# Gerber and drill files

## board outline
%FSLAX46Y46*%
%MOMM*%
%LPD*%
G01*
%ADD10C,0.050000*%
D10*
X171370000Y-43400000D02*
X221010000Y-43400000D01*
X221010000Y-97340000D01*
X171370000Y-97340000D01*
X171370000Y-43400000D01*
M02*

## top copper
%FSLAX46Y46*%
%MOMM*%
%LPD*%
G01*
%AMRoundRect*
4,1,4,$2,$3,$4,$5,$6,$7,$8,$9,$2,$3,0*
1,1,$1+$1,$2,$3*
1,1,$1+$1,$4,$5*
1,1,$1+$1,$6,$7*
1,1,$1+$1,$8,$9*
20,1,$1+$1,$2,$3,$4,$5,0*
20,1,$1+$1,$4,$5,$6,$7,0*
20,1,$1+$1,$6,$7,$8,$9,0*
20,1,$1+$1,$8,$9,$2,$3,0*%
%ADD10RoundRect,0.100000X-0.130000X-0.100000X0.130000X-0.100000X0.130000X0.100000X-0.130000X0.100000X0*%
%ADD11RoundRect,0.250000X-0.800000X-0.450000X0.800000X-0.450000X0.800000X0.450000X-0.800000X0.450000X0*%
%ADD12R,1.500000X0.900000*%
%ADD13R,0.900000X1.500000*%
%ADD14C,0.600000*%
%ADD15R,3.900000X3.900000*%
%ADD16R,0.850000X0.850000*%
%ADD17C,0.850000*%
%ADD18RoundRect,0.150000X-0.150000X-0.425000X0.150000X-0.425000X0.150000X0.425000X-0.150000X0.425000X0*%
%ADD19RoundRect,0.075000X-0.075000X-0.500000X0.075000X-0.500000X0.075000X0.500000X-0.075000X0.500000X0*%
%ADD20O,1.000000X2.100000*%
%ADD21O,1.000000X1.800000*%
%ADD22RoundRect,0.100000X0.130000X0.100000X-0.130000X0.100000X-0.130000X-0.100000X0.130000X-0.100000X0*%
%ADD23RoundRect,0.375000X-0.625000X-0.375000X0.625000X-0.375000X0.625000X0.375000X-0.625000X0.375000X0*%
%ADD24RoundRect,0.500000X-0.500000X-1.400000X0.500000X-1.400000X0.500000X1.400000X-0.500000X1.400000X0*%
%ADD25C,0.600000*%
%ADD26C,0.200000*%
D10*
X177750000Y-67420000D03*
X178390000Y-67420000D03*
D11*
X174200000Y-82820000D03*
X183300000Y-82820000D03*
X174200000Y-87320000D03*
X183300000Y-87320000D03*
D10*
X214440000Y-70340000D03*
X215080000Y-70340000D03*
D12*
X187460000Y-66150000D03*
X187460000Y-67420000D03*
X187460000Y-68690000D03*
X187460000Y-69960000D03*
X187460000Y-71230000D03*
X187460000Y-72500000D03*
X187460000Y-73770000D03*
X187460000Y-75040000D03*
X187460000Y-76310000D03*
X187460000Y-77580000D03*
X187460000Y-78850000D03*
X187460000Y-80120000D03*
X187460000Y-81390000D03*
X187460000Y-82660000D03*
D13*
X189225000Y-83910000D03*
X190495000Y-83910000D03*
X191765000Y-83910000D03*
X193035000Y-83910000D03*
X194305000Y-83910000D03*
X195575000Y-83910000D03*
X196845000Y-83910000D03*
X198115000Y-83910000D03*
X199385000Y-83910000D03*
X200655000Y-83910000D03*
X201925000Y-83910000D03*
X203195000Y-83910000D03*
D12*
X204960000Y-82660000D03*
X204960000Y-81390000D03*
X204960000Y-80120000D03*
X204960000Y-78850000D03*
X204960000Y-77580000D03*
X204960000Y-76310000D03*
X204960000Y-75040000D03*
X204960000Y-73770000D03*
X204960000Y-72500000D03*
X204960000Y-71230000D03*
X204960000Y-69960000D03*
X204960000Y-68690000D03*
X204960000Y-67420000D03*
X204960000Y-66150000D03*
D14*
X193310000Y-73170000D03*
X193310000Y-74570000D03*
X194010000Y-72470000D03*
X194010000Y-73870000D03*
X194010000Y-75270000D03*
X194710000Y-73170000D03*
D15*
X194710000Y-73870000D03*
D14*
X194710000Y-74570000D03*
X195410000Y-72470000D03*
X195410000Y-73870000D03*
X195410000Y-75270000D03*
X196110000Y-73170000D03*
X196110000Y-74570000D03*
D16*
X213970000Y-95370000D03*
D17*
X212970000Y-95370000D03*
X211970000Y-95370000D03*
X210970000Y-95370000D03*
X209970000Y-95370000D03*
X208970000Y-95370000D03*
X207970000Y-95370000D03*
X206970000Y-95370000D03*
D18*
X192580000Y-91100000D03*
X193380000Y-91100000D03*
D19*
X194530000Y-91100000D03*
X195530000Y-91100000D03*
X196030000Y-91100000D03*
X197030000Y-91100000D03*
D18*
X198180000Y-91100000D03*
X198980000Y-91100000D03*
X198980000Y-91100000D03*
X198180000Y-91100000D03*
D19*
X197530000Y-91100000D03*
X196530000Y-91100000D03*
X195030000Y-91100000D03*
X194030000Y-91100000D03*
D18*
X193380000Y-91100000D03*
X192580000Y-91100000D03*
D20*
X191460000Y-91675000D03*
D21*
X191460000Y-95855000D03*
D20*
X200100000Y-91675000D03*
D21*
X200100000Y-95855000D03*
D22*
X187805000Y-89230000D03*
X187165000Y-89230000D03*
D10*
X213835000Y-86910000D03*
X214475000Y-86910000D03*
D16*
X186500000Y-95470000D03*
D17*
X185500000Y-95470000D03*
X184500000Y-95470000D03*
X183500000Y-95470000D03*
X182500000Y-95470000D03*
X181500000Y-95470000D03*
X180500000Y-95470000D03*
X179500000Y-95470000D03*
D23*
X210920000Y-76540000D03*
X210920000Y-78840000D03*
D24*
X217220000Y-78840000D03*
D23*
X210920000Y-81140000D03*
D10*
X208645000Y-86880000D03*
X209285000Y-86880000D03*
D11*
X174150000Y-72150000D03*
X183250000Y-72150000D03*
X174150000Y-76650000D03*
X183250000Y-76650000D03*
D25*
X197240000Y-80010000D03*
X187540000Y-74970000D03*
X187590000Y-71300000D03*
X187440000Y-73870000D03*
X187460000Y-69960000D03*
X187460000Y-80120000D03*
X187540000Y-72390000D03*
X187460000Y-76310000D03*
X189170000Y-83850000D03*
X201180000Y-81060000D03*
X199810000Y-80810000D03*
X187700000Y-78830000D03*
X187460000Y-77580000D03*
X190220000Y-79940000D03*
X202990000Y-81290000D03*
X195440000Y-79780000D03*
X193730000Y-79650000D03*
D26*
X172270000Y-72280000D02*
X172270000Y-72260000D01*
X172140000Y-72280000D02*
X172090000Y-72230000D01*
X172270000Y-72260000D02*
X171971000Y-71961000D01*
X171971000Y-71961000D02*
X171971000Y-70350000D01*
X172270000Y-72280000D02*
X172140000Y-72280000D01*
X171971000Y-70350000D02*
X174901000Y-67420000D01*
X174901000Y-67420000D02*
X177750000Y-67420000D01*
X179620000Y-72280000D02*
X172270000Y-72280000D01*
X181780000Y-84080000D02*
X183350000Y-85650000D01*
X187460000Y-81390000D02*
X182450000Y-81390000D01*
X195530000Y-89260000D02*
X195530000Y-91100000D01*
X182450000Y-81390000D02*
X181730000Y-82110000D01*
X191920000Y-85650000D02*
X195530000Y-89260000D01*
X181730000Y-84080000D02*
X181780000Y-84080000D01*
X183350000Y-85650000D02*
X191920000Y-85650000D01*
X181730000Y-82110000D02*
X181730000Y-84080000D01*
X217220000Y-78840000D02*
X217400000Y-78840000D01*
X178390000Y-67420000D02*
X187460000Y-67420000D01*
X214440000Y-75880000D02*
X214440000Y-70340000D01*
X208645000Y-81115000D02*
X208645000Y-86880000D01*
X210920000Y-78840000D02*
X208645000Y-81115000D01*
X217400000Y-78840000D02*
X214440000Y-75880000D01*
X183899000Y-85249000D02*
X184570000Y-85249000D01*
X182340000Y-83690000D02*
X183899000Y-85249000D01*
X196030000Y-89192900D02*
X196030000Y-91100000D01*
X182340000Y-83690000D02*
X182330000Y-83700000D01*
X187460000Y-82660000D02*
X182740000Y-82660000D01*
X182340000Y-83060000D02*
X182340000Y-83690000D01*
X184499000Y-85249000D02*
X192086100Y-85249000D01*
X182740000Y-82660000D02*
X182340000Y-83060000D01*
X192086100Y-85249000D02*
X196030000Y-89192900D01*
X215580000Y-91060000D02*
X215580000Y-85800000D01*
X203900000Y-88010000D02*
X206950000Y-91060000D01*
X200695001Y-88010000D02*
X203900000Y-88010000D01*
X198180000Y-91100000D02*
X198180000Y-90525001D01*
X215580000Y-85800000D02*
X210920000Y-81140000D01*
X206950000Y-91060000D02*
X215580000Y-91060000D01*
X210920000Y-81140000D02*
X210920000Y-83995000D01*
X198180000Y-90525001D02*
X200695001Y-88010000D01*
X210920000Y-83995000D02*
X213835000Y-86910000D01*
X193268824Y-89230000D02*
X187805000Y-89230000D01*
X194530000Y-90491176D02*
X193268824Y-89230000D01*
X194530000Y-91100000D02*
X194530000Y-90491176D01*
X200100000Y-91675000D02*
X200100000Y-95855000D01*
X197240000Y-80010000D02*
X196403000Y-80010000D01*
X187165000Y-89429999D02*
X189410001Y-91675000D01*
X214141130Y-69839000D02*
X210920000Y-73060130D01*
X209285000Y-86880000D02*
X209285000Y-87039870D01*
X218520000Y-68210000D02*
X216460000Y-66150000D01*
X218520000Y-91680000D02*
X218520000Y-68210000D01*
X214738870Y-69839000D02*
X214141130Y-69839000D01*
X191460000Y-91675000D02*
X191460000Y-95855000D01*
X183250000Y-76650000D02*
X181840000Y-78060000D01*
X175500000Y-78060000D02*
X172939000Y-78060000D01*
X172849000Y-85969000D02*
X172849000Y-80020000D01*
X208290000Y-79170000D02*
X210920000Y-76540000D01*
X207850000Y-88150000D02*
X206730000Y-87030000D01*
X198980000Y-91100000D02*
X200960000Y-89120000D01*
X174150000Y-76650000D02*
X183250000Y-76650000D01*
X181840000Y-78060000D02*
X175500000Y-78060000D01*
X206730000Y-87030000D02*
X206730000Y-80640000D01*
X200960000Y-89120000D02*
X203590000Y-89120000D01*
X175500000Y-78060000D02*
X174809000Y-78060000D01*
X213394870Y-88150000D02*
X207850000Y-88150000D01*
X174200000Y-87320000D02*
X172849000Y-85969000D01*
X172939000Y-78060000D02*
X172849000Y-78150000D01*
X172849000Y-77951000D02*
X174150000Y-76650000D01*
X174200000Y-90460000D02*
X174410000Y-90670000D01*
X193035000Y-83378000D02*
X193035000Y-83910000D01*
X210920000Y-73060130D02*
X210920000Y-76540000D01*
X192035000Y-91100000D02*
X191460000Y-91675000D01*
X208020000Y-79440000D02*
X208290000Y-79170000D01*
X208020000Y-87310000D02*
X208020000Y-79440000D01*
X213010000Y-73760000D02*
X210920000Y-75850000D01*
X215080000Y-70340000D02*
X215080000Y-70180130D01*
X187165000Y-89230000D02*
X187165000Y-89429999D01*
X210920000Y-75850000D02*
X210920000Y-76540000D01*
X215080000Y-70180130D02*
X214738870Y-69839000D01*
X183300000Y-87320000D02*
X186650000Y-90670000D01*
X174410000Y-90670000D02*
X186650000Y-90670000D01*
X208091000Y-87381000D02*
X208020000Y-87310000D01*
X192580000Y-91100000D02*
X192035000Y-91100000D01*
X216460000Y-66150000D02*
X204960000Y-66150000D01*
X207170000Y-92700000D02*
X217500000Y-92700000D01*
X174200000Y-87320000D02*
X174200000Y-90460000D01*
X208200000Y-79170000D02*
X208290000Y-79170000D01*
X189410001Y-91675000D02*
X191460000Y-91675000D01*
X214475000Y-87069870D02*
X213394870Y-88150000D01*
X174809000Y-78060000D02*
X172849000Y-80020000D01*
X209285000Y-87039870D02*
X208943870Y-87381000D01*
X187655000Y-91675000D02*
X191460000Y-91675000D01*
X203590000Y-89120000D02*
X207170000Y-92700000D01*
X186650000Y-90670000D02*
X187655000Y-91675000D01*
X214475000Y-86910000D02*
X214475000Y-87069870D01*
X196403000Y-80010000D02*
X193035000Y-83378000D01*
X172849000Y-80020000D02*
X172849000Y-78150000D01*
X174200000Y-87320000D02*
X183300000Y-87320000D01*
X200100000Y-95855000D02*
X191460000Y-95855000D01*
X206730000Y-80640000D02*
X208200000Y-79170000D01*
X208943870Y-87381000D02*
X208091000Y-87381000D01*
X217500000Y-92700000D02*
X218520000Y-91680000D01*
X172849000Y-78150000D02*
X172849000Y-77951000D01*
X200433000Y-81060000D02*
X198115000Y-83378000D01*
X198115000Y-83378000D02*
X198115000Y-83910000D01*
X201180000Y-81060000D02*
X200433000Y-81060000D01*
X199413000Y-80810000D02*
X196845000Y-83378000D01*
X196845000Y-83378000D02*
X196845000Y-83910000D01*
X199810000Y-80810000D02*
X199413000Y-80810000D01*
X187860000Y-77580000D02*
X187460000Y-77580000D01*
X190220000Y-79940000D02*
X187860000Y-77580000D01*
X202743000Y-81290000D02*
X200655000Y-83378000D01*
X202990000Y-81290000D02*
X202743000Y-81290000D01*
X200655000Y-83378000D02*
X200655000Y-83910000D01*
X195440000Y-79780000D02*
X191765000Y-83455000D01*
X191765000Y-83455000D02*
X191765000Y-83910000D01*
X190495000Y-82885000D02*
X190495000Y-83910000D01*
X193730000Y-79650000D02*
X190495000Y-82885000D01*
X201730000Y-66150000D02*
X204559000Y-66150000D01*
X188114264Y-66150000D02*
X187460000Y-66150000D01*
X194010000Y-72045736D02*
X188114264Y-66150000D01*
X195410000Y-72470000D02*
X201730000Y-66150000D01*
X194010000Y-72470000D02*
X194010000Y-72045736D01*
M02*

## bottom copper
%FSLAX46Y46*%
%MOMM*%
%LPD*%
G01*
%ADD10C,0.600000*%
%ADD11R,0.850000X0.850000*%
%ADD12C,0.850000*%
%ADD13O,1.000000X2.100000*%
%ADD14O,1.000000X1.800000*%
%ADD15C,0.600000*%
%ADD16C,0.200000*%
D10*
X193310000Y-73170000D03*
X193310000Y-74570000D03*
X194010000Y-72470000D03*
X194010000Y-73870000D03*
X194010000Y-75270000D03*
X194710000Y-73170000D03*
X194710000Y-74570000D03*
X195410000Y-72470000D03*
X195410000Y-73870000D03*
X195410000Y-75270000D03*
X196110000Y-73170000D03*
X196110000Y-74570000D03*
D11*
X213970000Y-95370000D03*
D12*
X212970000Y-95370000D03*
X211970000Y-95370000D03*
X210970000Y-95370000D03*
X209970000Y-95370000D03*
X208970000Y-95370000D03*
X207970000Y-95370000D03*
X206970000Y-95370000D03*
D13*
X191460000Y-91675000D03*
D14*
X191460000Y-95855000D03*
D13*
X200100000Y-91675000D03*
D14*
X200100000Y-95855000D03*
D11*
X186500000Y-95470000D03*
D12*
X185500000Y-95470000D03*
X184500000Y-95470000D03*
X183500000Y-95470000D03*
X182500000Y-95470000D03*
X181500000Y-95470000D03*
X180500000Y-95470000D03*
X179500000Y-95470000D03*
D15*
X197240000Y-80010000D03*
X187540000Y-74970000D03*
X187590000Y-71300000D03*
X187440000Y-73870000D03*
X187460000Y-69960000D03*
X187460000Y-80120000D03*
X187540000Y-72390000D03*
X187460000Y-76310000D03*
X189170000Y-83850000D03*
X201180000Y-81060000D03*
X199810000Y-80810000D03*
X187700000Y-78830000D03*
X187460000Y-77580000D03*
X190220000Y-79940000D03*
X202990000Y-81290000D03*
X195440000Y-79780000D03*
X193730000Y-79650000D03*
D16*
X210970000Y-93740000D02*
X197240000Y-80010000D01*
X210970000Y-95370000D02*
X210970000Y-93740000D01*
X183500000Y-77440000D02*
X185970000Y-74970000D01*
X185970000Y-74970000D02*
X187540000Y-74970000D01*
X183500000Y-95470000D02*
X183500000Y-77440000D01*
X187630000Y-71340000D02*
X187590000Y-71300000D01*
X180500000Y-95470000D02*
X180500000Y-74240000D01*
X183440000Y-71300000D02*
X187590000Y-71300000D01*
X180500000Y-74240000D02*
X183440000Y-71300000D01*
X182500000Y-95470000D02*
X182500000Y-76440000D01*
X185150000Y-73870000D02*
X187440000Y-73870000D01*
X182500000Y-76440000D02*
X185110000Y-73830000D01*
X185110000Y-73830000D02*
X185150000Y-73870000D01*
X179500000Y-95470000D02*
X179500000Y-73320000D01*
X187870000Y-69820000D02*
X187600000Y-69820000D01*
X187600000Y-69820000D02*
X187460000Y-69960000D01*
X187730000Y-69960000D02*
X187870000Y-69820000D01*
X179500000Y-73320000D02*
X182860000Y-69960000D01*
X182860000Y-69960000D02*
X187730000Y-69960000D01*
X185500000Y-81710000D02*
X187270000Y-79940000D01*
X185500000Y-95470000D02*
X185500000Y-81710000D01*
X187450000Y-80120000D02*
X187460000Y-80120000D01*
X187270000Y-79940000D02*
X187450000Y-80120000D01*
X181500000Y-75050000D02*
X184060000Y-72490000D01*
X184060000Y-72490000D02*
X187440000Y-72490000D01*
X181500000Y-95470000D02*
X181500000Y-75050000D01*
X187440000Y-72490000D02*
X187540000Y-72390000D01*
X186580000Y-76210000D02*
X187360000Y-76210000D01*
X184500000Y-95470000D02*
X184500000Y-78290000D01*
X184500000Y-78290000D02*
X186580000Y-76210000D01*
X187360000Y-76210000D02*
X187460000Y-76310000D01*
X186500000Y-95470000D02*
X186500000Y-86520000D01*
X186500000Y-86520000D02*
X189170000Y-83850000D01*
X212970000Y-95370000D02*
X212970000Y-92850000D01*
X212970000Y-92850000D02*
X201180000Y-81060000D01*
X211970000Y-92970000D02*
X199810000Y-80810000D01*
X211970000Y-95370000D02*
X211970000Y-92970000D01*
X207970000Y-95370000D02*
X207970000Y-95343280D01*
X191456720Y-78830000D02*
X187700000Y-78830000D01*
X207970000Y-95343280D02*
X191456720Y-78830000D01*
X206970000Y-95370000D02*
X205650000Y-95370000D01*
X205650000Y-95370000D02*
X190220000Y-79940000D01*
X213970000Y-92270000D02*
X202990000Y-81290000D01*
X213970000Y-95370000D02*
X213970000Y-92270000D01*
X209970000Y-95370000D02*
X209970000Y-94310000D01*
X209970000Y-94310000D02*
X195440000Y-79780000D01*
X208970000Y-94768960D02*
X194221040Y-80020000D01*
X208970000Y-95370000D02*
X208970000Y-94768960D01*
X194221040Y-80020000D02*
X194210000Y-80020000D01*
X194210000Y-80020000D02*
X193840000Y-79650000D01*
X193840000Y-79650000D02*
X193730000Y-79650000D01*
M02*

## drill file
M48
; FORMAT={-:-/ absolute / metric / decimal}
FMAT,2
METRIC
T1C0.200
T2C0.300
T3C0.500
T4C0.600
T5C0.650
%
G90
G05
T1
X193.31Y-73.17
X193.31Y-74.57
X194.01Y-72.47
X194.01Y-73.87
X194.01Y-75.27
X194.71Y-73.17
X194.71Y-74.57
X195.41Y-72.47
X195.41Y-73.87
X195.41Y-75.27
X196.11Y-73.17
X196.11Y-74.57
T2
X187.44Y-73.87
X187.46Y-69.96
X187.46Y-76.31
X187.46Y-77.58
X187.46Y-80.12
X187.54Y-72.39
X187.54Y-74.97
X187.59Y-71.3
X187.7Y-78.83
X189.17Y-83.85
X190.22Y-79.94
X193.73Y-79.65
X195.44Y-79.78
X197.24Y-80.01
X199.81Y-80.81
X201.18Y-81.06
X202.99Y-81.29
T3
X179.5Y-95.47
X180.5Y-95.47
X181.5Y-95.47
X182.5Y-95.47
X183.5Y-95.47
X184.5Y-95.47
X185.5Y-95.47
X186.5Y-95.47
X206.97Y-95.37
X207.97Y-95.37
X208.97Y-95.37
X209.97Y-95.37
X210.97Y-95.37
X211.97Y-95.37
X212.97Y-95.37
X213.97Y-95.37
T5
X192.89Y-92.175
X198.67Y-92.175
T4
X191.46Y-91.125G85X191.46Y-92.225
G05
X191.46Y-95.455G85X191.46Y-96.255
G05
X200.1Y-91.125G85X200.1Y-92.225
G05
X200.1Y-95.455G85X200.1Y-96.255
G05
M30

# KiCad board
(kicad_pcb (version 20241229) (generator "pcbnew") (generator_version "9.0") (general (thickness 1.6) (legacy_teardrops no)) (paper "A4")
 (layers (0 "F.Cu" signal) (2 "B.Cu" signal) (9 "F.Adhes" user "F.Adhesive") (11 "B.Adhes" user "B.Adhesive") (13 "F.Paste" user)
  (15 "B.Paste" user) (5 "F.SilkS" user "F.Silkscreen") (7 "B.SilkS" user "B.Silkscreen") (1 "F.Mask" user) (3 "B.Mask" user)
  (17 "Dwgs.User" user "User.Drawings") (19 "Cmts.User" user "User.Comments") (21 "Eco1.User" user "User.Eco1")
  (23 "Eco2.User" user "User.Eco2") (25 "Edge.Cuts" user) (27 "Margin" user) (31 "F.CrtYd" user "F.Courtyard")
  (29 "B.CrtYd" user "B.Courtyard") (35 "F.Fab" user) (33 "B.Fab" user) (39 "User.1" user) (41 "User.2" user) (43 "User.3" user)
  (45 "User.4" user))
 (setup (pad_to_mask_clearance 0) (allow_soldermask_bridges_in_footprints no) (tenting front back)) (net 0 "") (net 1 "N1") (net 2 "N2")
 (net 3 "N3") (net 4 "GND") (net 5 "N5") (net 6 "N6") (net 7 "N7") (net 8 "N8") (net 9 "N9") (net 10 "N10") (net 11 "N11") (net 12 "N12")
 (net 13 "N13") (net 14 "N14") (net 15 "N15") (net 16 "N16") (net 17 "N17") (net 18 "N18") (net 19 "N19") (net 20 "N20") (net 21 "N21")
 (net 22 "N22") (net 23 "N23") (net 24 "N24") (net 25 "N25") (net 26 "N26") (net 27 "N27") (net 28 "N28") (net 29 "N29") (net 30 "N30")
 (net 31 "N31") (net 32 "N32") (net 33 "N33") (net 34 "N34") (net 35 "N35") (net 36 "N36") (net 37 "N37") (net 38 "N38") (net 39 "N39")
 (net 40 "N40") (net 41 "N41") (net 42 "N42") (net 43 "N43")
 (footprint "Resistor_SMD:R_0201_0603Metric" (layer "F.Cu") (at 178.07 67.42)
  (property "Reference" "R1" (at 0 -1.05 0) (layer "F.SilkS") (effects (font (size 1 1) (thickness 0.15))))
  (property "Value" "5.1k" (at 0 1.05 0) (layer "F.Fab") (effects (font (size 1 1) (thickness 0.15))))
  (pad "" smd roundrect (at -0.345 0) (size 0.318 0.36) (layers "F.Paste") (roundrect_rratio 0.25))
  (pad "" smd roundrect (at 0.345 0) (size 0.318 0.36) (layers "F.Paste") (roundrect_rratio 0.25))
  (pad "1" smd roundrect (at -0.32 0) (size 0.46 0.4) (layers "F.Cu" "F.Mask") (roundrect_rratio 0.25) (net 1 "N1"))
  (pad "2" smd roundrect (at 0.32 0) (size 0.46 0.4) (layers "F.Cu" "F.Mask") (roundrect_rratio 0.25) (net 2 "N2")))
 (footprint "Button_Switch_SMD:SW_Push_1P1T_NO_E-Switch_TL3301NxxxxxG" (layer "F.Cu") (at 178.75 85.07)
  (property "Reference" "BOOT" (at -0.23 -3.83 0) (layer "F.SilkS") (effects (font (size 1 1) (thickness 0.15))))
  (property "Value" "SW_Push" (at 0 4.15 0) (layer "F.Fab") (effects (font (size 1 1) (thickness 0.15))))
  (pad "1" smd roundrect (at -4.55 -2.25) (size 2.1 1.4) (layers "F.Cu" "F.Mask" "F.Paste") (roundrect_rratio 0.1785714286) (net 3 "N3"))
  (pad "1" smd roundrect (at 4.55 -2.25) (size 2.1 1.4) (layers "F.Cu" "F.Mask" "F.Paste") (roundrect_rratio 0.1785714286) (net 3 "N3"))
  (pad "2" smd roundrect (at -4.55 2.25) (size 2.1 1.4) (layers "F.Cu" "F.Mask" "F.Paste") (roundrect_rratio 0.1785714286) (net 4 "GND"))
  (pad "2" smd roundrect (at 4.55 2.25) (size 2.1 1.4) (layers "F.Cu" "F.Mask" "F.Paste") (roundrect_rratio 0.1785714286) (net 4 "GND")))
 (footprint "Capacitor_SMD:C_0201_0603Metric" (layer "F.Cu") (at 214.76 70.34)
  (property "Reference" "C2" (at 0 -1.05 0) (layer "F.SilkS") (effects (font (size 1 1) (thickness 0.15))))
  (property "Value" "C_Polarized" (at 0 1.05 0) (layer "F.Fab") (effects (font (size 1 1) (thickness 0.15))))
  (pad "" smd roundrect (at -0.345 0) (size 0.318 0.36) (layers "F.Paste") (roundrect_rratio 0.25))
  (pad "" smd roundrect (at 0.345 0) (size 0.318 0.36) (layers "F.Paste") (roundrect_rratio 0.25))
  (pad "1" smd roundrect (at -0.32 0) (size 0.46 0.4) (layers "F.Cu" "F.Mask") (roundrect_rratio 0.25) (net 2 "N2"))
  (pad "2" smd roundrect (at 0.32 0) (size 0.46 0.4) (layers "F.Cu" "F.Mask") (roundrect_rratio 0.25) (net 4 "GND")))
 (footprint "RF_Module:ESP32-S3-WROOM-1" (layer "F.Cu") (at 196.21 71.41)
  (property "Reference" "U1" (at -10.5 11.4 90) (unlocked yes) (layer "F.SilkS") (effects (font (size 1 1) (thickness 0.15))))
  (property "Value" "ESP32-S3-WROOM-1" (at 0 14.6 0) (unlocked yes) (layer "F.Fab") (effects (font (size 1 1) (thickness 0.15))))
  (pad "" smd rect (at -2.9 1.06) (size 0.9 0.9) (layers "F.Paste"))
  (pad "" smd rect (at -2.9 2.46 270) (size 0.9 0.9) (layers "F.Paste"))
  (pad "" smd rect (at -2.9 3.86) (size 0.9 0.9) (layers "F.Paste"))
  (pad "" smd rect (at -1.5 1.06 270) (size 0.9 0.9) (layers "F.Paste"))
  (pad "" smd rect (at -1.5 2.46 270) (size 0.9 0.9) (layers "F.Paste"))
  (pad "" smd rect (at -1.5 3.86 270) (size 0.9 0.9) (layers "F.Paste"))
  (pad "" smd rect (at -0.1 1.06 270) (size 0.9 0.9) (layers "F.Paste"))
  (pad "" smd rect (at -0.1 2.46 270) (size 0.9 0.9) (layers "F.Paste"))
  (pad "" smd rect (at -0.1 3.86 270) (size 0.9 0.9) (layers "F.Paste"))
  (pad "1" smd rect (at -8.75 -5.26) (size 1.5 0.9) (layers "F.Cu" "F.Mask" "F.Paste") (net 4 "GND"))
  (pad "2" smd rect (at -8.75 -3.99) (size 1.5 0.9) (layers "F.Cu" "F.Mask" "F.Paste") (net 2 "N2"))
  (pad "3" smd rect (at -8.75 -2.72) (size 1.5 0.9) (layers "F.Cu" "F.Mask" "F.Paste") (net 1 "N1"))
  (pad "4" smd rect (at -8.75 -1.45) (size 1.5 0.9) (layers "F.Cu" "F.Mask" "F.Paste") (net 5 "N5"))
  (pad "5" smd rect (at -8.75 -0.18) (size 1.5 0.9) (layers "F.Cu" "F.Mask" "F.Paste") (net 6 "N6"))
  (pad "6" smd rect (at -8.75 1.09) (size 1.5 0.9) (layers "F.Cu" "F.Mask" "F.Paste") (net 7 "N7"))
  (pad "7" smd rect (at -8.75 2.36) (size 1.5 0.9) (layers "F.Cu" "F.Mask" "F.Paste") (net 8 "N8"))
  (pad "8" smd rect (at -8.75 3.63) (size 1.5 0.9) (layers "F.Cu" "F.Mask" "F.Paste") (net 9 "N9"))
  (pad "9" smd rect (at -8.75 4.9) (size 1.5 0.9) (layers "F.Cu" "F.Mask" "F.Paste") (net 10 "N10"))
  (pad "10" smd rect (at -8.75 6.17) (size 1.5 0.9) (layers "F.Cu" "F.Mask" "F.Paste") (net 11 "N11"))
  (pad "11" smd rect (at -8.75 7.44) (size 1.5 0.9) (layers "F.Cu" "F.Mask" "F.Paste") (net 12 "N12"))
  (pad "12" smd rect (at -8.75 8.71) (size 1.5 0.9) (layers "F.Cu" "F.Mask" "F.Paste") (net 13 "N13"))
  (pad "13" smd rect (at -8.75 9.98) (size 1.5 0.9) (layers "F.Cu" "F.Mask" "F.Paste") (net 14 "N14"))
  (pad "14" smd rect (at -8.75 11.25 180) (size 1.5 0.9) (layers "F.Cu" "F.Mask" "F.Paste") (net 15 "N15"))
  (pad "15" smd rect (at -6.985 12.5 270) (size 1.5 0.9) (layers "F.Cu" "F.Mask" "F.Paste") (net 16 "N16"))
  (pad "16" smd rect (at -5.715 12.5 270) (size 1.5 0.9) (layers "F.Cu" "F.Mask" "F.Paste") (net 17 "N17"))
  (pad "17" smd rect (at -4.445 12.5 270) (size 1.5 0.9) (layers "F.Cu" "F.Mask" "F.Paste") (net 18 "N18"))
  (pad "18" smd rect (at -3.175 12.5 270) (size 1.5 0.9) (layers "F.Cu" "F.Mask" "F.Paste") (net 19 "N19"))
  (pad "19" smd rect (at -1.905 12.5 270) (size 1.5 0.9) (layers "F.Cu" "F.Mask" "F.Paste") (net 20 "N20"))
  (pad "20" smd rect (at -0.635 12.5 270) (size 1.5 0.9) (layers "F.Cu" "F.Mask" "F.Paste") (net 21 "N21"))
  (pad "21" smd rect (at 0.635 12.5 270) (size 1.5 0.9) (layers "F.Cu" "F.Mask" "F.Paste") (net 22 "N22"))
  (pad "22" smd rect (at 1.905 12.5 270) (size 1.5 0.9) (layers "F.Cu" "F.Mask" "F.Paste") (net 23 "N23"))
  (pad "23" smd rect (at 3.175 12.5 270) (size 1.5 0.9) (layers "F.Cu" "F.Mask" "F.Paste") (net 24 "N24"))
  (pad "24" smd rect (at 4.445 12.5 270) (size 1.5 0.9) (layers "F.Cu" "F.Mask" "F.Paste") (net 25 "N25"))
  (pad "25" smd rect (at 5.715 12.5 270) (size 1.5 0.9) (layers "F.Cu" "F.Mask" "F.Paste") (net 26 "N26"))
  (pad "26" smd rect (at 6.985 12.5 270) (size 1.5 0.9) (layers "F.Cu" "F.Mask" "F.Paste") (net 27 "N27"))
  (pad "27" smd rect (at 8.75 11.25) (size 1.5 0.9) (layers "F.Cu" "F.Mask" "F.Paste") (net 3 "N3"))
  (pad "28" smd rect (at 8.75 9.98) (size 1.5 0.9) (layers "F.Cu" "F.Mask" "F.Paste") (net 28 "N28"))
  (pad "29" smd rect (at 8.75 8.71) (size 1.5 0.9) (layers "F.Cu" "F.Mask" "F.Paste") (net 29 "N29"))
  (pad "30" smd rect (at 8.75 7.44) (size 1.5 0.9) (layers "F.Cu" "F.Mask" "F.Paste") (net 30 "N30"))
  (pad "31" smd rect (at 8.75 6.17) (size 1.5 0.9) (layers "F.Cu" "F.Mask" "F.Paste") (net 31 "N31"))
  (pad "32" smd rect (at 8.75 4.9) (size 1.5 0.9) (layers "F.Cu" "F.Mask" "F.Paste") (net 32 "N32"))
  (pad "33" smd rect (at 8.75 3.63) (size 1.5 0.9) (layers "F.Cu" "F.Mask" "F.Paste") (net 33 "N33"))
  (pad "34" smd rect (at 8.75 2.36) (size 1.5 0.9) (layers "F.Cu" "F.Mask" "F.Paste") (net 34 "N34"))
  (pad "35" smd rect (at 8.75 1.09) (size 1.5 0.9) (layers "F.Cu" "F.Mask" "F.Paste") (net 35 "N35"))
  (pad "36" smd rect (at 8.75 -0.18) (size 1.5 0.9) (layers "F.Cu" "F.Mask" "F.Paste") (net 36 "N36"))
  (pad "37" smd rect (at 8.75 -1.45) (size 1.5 0.9) (layers "F.Cu" "F.Mask" "F.Paste") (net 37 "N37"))
  (pad "38" smd rect (at 8.75 -2.72) (size 1.5 0.9) (layers "F.Cu" "F.Mask" "F.Paste") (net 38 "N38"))
  (pad "39" smd rect (at 8.75 -3.99) (size 1.5 0.9) (layers "F.Cu" "F.Mask" "F.Paste") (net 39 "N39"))
  (pad "40" smd rect (at 8.75 -5.26) (size 1.5 0.9) (layers "F.Cu" "F.Mask" "F.Paste") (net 4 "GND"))
  (pad "41" thru_hole circle (at -2.9 1.76 90) (size 0.6 0.6) (drill 0.2) (layers "*.Cu" "F.Mask") (remove_unused_layers no) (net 4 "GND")
   (zone_connect 2))
  (pad "41" thru_hole circle (at -2.9 3.16) (size 0.6 0.6) (drill 0.2) (layers "*.Cu" "F.Mask") (remove_unused_layers no) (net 4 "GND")
   (zone_connect 2))
  (pad "41" thru_hole circle (at -2.2 1.06) (size 0.6 0.6) (drill 0.2) (layers "*.Cu" "F.Mask") (remove_unused_layers no) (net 4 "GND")
   (zone_connect 2))
  (pad "41" thru_hole circle (at -2.2 2.46) (size 0.6 0.6) (drill 0.2) (layers "*.Cu" "F.Mask") (remove_unused_layers no) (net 4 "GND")
   (zone_connect 2))
  (pad "41" thru_hole circle (at -2.2 3.86) (size 0.6 0.6) (drill 0.2) (layers "*.Cu" "F.Mask") (remove_unused_layers no) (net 4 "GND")
   (zone_connect 2))
  (pad "41" thru_hole circle (at -1.5 1.76) (size 0.6 0.6) (drill 0.2) (layers "*.Cu" "F.Mask") (remove_unused_layers no) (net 4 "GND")
   (zone_connect 2))
  (pad "41" smd rect (at -1.5 2.46 270) (size 3.9 3.9) (layers "F.Cu" "F.Mask") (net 4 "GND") (zone_connect 2))
  (pad "41" thru_hole circle (at -1.5 3.16) (size 0.6 0.6) (drill 0.2) (layers "*.Cu" "F.Mask") (remove_unused_layers no) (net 4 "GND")
   (zone_connect 2))
  (pad "41" thru_hole circle (at -0.8 1.06) (size 0.6 0.6) (drill 0.2) (layers "*.Cu" "F.Mask") (remove_unused_layers no) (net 4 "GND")
   (zone_connect 2))
  (pad "41" thru_hole circle (at -0.8 2.46) (size 0.6 0.6) (drill 0.2) (layers "*.Cu" "F.Mask") (remove_unused_layers no) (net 4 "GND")
   (zone_connect 2))
  (pad "41" thru_hole circle (at -0.8 3.86) (size 0.6 0.6) (drill 0.2) (layers "*.Cu" "F.Mask") (remove_unused_layers no) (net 4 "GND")
   (zone_connect 2))
  (pad "41" thru_hole circle (at -0.1 1.76) (size 0.6 0.6) (drill 0.2) (layers "*.Cu" "F.Mask") (remove_unused_layers no) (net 4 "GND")
   (zone_connect 2))
  (pad "41" thru_hole circle (at -0.1 3.16) (size 0.6 0.6) (drill 0.2) (layers "*.Cu" "F.Mask") (remove_unused_layers no) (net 4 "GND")
   (zone_connect 2))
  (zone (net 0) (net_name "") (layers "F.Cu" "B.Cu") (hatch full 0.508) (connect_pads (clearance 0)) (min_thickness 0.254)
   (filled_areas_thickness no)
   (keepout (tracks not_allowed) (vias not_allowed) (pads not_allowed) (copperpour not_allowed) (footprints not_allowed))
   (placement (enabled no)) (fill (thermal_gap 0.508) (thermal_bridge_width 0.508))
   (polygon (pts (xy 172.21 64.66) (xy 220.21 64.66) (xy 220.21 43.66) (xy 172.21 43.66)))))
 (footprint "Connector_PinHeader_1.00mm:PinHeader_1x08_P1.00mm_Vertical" (layer "F.Cu") (at 213.97 95.37 -90)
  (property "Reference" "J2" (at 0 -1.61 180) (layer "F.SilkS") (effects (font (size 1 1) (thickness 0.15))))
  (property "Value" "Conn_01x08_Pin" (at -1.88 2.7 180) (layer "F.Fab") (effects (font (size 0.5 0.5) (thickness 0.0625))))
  (pad "1" thru_hole rect (at 0 0 270) (size 0.85 0.85) (drill 0.5) (layers "*.Cu" "*.Mask") (remove_unused_layers no) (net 25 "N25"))
  (pad "2" thru_hole circle (at 0 1 270) (size 0.85 0.85) (drill 0.5) (layers "*.Cu" "*.Mask") (remove_unused_layers no) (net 23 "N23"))
  (pad "3" thru_hole circle (at 0 2 270) (size 0.85 0.85) (drill 0.5) (layers "*.Cu" "*.Mask") (remove_unused_layers no) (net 22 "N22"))
  (pad "4" thru_hole circle (at 0 3 270) (size 0.85 0.85) (drill 0.5) (layers "*.Cu" "*.Mask") (remove_unused_layers no) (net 19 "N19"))
  (pad "5" thru_hole circle (at 0 4 270) (size 0.85 0.85) (drill 0.5) (layers "*.Cu" "*.Mask") (remove_unused_layers no) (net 18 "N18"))
  (pad "6" thru_hole circle (at 0 5 270) (size 0.85 0.85) (drill 0.5) (layers "*.Cu" "*.Mask") (remove_unused_layers no) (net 17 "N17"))
  (pad "7" thru_hole circle (at 0 6 270) (size 0.85 0.85) (drill 0.5) (layers "*.Cu" "*.Mask") (remove_unused_layers no) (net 12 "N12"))
  (pad "8" thru_hole circle (at 0 7 270) (size 0.85 0.85) (drill 0.5) (layers "*.Cu" "*.Mask") (remove_unused_layers no) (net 11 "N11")))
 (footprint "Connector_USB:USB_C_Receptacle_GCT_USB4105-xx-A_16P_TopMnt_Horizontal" (layer "F.Cu") (at 195.78 94.78)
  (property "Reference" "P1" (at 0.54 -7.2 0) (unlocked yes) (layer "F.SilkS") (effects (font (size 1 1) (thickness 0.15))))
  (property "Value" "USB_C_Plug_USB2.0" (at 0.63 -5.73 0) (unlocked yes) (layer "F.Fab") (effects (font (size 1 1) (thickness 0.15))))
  (pad "" np_thru_hole circle (at -2.89 -2.605) (size 0.65 0.65) (drill 0.65) (layers "*.Cu" "*.Mask"))
  (pad "" np_thru_hole circle (at 2.89 -2.605) (size 0.65 0.65) (drill 0.65) (layers "*.Cu" "*.Mask"))
  (pad "A1" smd roundrect (at -3.2 -3.68) (size 0.6 1.15) (layers "F.Cu" "F.Mask" "F.Paste") (roundrect_rratio 0.25) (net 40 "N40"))
  (pad "A4" smd roundrect (at -2.4 -3.68) (size 0.6 1.15) (layers "F.Cu" "F.Mask" "F.Paste") (roundrect_rratio 0.25) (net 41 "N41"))
  (pad "A5" smd roundrect (at -1.25 -3.68) (size 0.3 1.15) (layers "F.Cu" "F.Mask" "F.Paste") (roundrect_rratio 0.25) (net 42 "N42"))
  (pad "A6" smd roundrect (at -0.25 -3.68) (size 0.3 1.15) (layers "F.Cu" "F.Mask" "F.Paste") (roundrect_rratio 0.25) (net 14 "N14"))
  (pad "A7" smd roundrect (at 0.25 -3.68) (size 0.3 1.15) (layers "F.Cu" "F.Mask" "F.Paste") (roundrect_rratio 0.25) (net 15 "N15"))
  (pad "A8" smd roundrect (at 1.25 -3.68) (size 0.3 1.15) (layers "F.Cu" "F.Mask" "F.Paste") (roundrect_rratio 0.25))
  (pad "A9" smd roundrect (at 2.4 -3.68) (size 0.6 1.15) (layers "F.Cu" "F.Mask" "F.Paste") (roundrect_rratio 0.25) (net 41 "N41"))
  (pad "A12" smd roundrect (at 3.2 -3.68) (size 0.6 1.15) (layers "F.Cu" "F.Mask" "F.Paste") (roundrect_rratio 0.25) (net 40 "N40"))
  (pad "B1" smd roundrect (at 3.2 -3.68) (size 0.6 1.15) (layers "F.Cu" "F.Mask" "F.Paste") (roundrect_rratio 0.25) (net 40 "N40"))
  (pad "B4" smd roundrect (at 2.4 -3.68) (size 0.6 1.15) (layers "F.Cu" "F.Mask" "F.Paste") (roundrect_rratio 0.25) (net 41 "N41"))
  (pad "B5" smd roundrect (at 1.75 -3.68) (size 0.3 1.15) (layers "F.Cu" "F.Mask" "F.Paste") (roundrect_rratio 0.25) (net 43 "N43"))
  (pad "B6" smd roundrect (at 0.75 -3.68) (size 0.3 1.15) (layers "F.Cu" "F.Mask" "F.Paste") (roundrect_rratio 0.25))
  (pad "B7" smd roundrect (at -0.75 -3.68) (size 0.3 1.15) (layers "F.Cu" "F.Mask" "F.Paste") (roundrect_rratio 0.25))
  (pad "B8" smd roundrect (at -1.75 -3.68) (size 0.3 1.15) (layers "F.Cu" "F.Mask" "F.Paste") (roundrect_rratio 0.25))
  (pad "B9" smd roundrect (at -2.4 -3.68) (size 0.6 1.15) (layers "F.Cu" "F.Mask" "F.Paste") (roundrect_rratio 0.25) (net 41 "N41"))
  (pad "B12" smd roundrect (at -3.2 -3.68) (size 0.6 1.15) (layers "F.Cu" "F.Mask" "F.Paste") (roundrect_rratio 0.25) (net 40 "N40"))
  (pad "S1" thru_hole oval (at -4.32 -3.105) (size 1 2.1) (drill oval 0.6 1.7) (layers "*.Cu" "*.Mask" "F.Paste") (remove_unused_layers no)
   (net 40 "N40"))
  (pad "S1" thru_hole oval (at -4.32 1.075) (size 1 1.8) (drill oval 0.6 1.4) (layers "*.Cu" "*.Mask" "F.Paste") (remove_unused_layers no)
   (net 40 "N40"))
  (pad "S1" thru_hole oval (at 4.32 -3.105) (size 1 2.1) (drill oval 0.6 1.7) (layers "*.Cu" "*.Mask" "F.Paste") (remove_unused_layers no)
   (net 40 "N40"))
  (pad "S1" thru_hole oval (at 4.32 1.075) (size 1 1.8) (drill oval 0.6 1.4) (layers "*.Cu" "*.Mask" "F.Paste") (remove_unused_layers no)
   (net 40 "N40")))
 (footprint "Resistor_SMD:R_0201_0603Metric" (layer "F.Cu") (at 187.485 89.23 180)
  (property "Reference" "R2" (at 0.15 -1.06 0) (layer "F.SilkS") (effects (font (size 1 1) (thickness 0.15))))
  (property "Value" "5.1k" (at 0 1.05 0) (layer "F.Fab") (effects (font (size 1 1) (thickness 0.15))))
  (pad "" smd roundrect (at -0.345 0 180) (size 0.318 0.36) (layers "F.Paste") (roundrect_rratio 0.25))
  (pad "" smd roundrect (at 0.345 0 180) (size 0.318 0.36) (layers "F.Paste") (roundrect_rratio 0.25))
  (pad "1" smd roundrect (at -0.32 0 180) (size 0.46 0.4) (layers "F.Cu" "F.Mask") (roundrect_rratio 0.25) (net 42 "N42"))
  (pad "2" smd roundrect (at 0.32 0 180) (size 0.46 0.4) (layers "F.Cu" "F.Mask") (roundrect_rratio 0.25) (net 4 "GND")))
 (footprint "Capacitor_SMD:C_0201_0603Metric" (layer "F.Cu") (at 214.155 86.91)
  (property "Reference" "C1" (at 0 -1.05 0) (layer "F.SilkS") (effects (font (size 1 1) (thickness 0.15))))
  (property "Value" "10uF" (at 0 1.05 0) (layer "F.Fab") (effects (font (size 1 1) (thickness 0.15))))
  (pad "" smd roundrect (at -0.345 0) (size 0.318 0.36) (layers "F.Paste") (roundrect_rratio 0.25))
  (pad "" smd roundrect (at 0.345 0) (size 0.318 0.36) (layers "F.Paste") (roundrect_rratio 0.25))
  (pad "1" smd roundrect (at -0.32 0) (size 0.46 0.4) (layers "F.Cu" "F.Mask") (roundrect_rratio 0.25) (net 41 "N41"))
  (pad "2" smd roundrect (at 0.32 0) (size 0.46 0.4) (layers "F.Cu" "F.Mask") (roundrect_rratio 0.25) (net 4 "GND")))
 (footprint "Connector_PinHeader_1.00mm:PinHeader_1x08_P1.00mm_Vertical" (layer "F.Cu") (at 186.5 95.47 -90)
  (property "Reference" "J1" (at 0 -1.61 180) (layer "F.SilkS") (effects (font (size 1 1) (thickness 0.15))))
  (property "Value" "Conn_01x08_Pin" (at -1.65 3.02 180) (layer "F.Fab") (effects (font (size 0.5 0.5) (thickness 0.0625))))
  (pad "1" thru_hole rect (at 0 0 270) (size 0.85 0.85) (drill 0.5) (layers "*.Cu" "*.Mask") (remove_unused_layers no) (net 16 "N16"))
  (pad "2" thru_hole circle (at 0 1 270) (size 0.85 0.85) (drill 0.5) (layers "*.Cu" "*.Mask") (remove_unused_layers no) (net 13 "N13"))
  (pad "3" thru_hole circle (at 0 2 270) (size 0.85 0.85) (drill 0.5) (layers "*.Cu" "*.Mask") (remove_unused_layers no) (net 10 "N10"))
  (pad "4" thru_hole circle (at 0 3 270) (size 0.85 0.85) (drill 0.5) (layers "*.Cu" "*.Mask") (remove_unused_layers no) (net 9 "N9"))
  (pad "5" thru_hole circle (at 0 4 270) (size 0.85 0.85) (drill 0.5) (layers "*.Cu" "*.Mask") (remove_unused_layers no) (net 8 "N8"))
  (pad "6" thru_hole circle (at 0 5 270) (size 0.85 0.85) (drill 0.5) (layers "*.Cu" "*.Mask") (remove_unused_layers no) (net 7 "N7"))
  (pad "7" thru_hole circle (at 0 6 270) (size 0.85 0.85) (drill 0.5) (layers "*.Cu" "*.Mask") (remove_unused_layers no) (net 6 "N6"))
  (pad "8" thru_hole circle (at 0 7 270) (size 0.85 0.85) (drill 0.5) (layers "*.Cu" "*.Mask") (remove_unused_layers no) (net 5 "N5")))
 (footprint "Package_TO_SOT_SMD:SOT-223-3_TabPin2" (layer "F.Cu") (at 214.07 78.84)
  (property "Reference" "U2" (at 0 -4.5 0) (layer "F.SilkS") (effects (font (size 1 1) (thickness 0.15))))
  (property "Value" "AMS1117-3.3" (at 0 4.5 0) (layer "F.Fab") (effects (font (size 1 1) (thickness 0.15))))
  (pad "1" smd roundrect (at -3.15 -2.3) (size 2 1.5) (layers "F.Cu" "F.Mask" "F.Paste") (roundrect_rratio 0.25) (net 40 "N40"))
  (pad "2" smd roundrect (at -3.15 0) (size 2 1.5) (layers "F.Cu" "F.Mask" "F.Paste") (roundrect_rratio 0.25) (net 2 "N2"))
  (pad "2" smd roundrect (at 3.15 0) (size 2 3.8) (layers "F.Cu" "F.Mask" "F.Paste") (roundrect_rratio 0.25) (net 2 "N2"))
  (pad "3" smd roundrect (at -3.15 2.3) (size 2 1.5) (layers "F.Cu" "F.Mask" "F.Paste") (roundrect_rratio 0.25) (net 41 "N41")))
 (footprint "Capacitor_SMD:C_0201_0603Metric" (layer "F.Cu") (at 208.965 86.88)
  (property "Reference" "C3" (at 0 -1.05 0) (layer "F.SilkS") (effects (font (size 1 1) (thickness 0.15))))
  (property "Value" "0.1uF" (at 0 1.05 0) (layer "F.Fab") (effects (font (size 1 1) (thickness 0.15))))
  (pad "" smd roundrect (at -0.345 0) (size 0.318 0.36) (layers "F.Paste") (roundrect_rratio 0.25))
  (pad "" smd roundrect (at 0.345 0) (size 0.318 0.36) (layers "F.Paste") (roundrect_rratio 0.25))
  (pad "1" smd roundrect (at -0.32 0) (size 0.46 0.4) (layers "F.Cu" "F.Mask") (roundrect_rratio 0.25) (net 2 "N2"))
  (pad "2" smd roundrect (at 0.32 0) (size 0.46 0.4) (layers "F.Cu" "F.Mask") (roundrect_rratio 0.25) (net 40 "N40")))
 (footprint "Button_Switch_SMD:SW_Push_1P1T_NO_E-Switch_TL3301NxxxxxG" (layer "F.Cu") (at 178.7 74.4)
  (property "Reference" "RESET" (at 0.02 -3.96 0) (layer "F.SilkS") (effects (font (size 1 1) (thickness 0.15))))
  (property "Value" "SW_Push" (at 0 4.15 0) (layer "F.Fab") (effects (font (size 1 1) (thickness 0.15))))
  (pad "1" smd roundrect (at -4.55 -2.25) (size 2.1 1.4) (layers "F.Cu" "F.Mask" "F.Paste") (roundrect_rratio 0.1785714286) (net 1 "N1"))
  (pad "1" smd roundrect (at 4.55 -2.25) (size 2.1 1.4) (layers "F.Cu" "F.Mask" "F.Paste") (roundrect_rratio 0.1785714286) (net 1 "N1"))
  (pad "2" smd roundrect (at -4.55 2.25) (size 2.1 1.4) (layers "F.Cu" "F.Mask" "F.Paste") (roundrect_rratio 0.1785714286) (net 4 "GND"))
  (pad "2" smd roundrect (at 4.55 2.25) (size 2.1 1.4) (layers "F.Cu" "F.Mask" "F.Paste") (roundrect_rratio 0.1785714286) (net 4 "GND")))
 (gr_rect (start 171.37 43.4) (end 221.01 97.34) (stroke (width 0.05) (type default)) (fill no) (layer "Edge.Cuts"))
 (segment (start 172.27 72.28) (end 172.27 72.26) (width 0.2) (layer "F.Cu") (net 1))
 (segment (start 172.14 72.28) (end 172.09 72.23) (width 0.2) (layer "F.Cu") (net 1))
 (segment (start 172.27 72.26) (end 171.971 71.961) (width 0.2) (layer "F.Cu") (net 1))
 (segment (start 171.971 71.961) (end 171.971 70.35) (width 0.2) (layer "F.Cu") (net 1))
 (segment (start 172.27 72.28) (end 172.14 72.28) (width 0.2) (layer "F.Cu") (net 1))
 (segment (start 171.971 70.35) (end 174.901 67.42) (width 0.2) (layer "F.Cu") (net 1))
 (segment (start 174.901 67.42) (end 177.75 67.42) (width 0.2) (layer "F.Cu") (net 1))
 (segment (start 179.62 72.28) (end 172.27 72.28) (width 0.2) (layer "F.Cu") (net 1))
 (segment (start 181.78 84.08) (end 183.35 85.65) (width 0.2) (layer "F.Cu") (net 14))
 (segment (start 187.46 81.39) (end 182.45 81.39) (width 0.2) (layer "F.Cu") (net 14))
 (segment (start 195.53 89.26) (end 195.53 91.1) (width 0.2) (layer "F.Cu") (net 14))
 (segment (start 182.45 81.39) (end 181.73 82.11) (width 0.2) (layer "F.Cu") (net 14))
 (segment (start 191.92 85.65) (end 195.53 89.26) (width 0.2) (layer "F.Cu") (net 14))
 (segment (start 181.73 84.08) (end 181.78 84.08) (width 0.2) (layer "F.Cu") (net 14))
 (segment (start 183.35 85.65) (end 191.92 85.65) (width 0.2) (layer "F.Cu") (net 14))
 (segment (start 181.73 82.11) (end 181.73 84.08) (width 0.2) (layer "F.Cu") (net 14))
 (segment (start 217.22 78.84) (end 217.4 78.84) (width 0.2) (layer "F.Cu") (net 2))
 (segment (start 178.39 67.42) (end 187.46 67.42) (width 0.2) (layer "F.Cu") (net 2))
 (segment (start 214.44 75.88) (end 214.44 70.34) (width 0.2) (layer "F.Cu") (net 2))
 (segment (start 208.645 81.115) (end 208.645 86.88) (width 0.2) (layer "F.Cu") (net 2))
 (segment (start 210.92 78.84) (end 208.645 81.115) (width 0.2) (layer "F.Cu") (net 2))
 (segment (start 217.4 78.84) (end 214.44 75.88) (width 0.2) (layer "F.Cu") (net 2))
 (segment (start 183.899 85.249) (end 184.57 85.249) (width 0.2) (layer "F.Cu") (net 15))
 (segment (start 182.34 83.69) (end 183.899 85.249) (width 0.2) (layer "F.Cu") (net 15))
 (segment (start 196.03 89.1929) (end 196.03 91.1) (width 0.2) (layer "F.Cu") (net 15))
 (segment (start 182.34 83.69) (end 182.33 83.7) (width 0.2) (layer "F.Cu") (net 15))
 (segment (start 187.46 82.66) (end 182.74 82.66) (width 0.2) (layer "F.Cu") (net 15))
 (segment (start 182.34 83.06) (end 182.34 83.69) (width 0.2) (layer "F.Cu") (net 15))
 (segment (start 184.499 85.249) (end 192.0861 85.249) (width 0.2) (layer "F.Cu") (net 15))
 (segment (start 182.74 82.66) (end 182.34 83.06) (width 0.2) (layer "F.Cu") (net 15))
 (segment (start 192.0861 85.249) (end 196.03 89.1929) (width 0.2) (layer "F.Cu") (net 15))
 (segment (start 215.58 91.06) (end 215.58 85.8) (width 0.2) (layer "F.Cu") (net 41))
 (segment (start 203.9 88.01) (end 206.95 91.06) (width 0.2) (layer "F.Cu") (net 41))
 (segment (start 200.695001 88.01) (end 203.9 88.01) (width 0.2) (layer "F.Cu") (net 41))
 (segment (start 198.18 91.1) (end 198.18 90.525001) (width 0.2) (layer "F.Cu") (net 41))
 (segment (start 215.58 85.8) (end 210.92 81.14) (width 0.2) (layer "F.Cu") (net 41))
 (segment (start 206.95 91.06) (end 215.58 91.06) (width 0.2) (layer "F.Cu") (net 41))
 (segment (start 210.92 81.14) (end 210.92 83.995) (width 0.2) (layer "F.Cu") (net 41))
 (segment (start 198.18 90.525001) (end 200.695001 88.01) (width 0.2) (layer "F.Cu") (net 41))
 (segment (start 210.92 83.995) (end 213.835 86.91) (width 0.2) (layer "F.Cu") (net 41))
 (segment (start 193.268824 89.23) (end 187.805 89.23) (width 0.2) (layer "F.Cu") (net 42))
 (segment (start 194.53 90.491176) (end 193.268824 89.23) (width 0.2) (layer "F.Cu") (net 42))
 (segment (start 194.53 91.1) (end 194.53 90.491176) (width 0.2) (layer "F.Cu") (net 42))
 (segment (start 200.1 91.675) (end 200.1 95.855) (width 0.2) (layer "F.Cu") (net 19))
 (segment (start 197.24 80.01) (end 196.403 80.01) (width 0.2) (layer "F.Cu") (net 19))
 (segment (start 187.165 89.429999) (end 189.410001 91.675) (width 0.2) (layer "F.Cu") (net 19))
 (segment (start 214.14113 69.839) (end 210.92 73.06013) (width 0.2) (layer "F.Cu") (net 19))
 (segment (start 209.285 86.88) (end 209.285 87.03987) (width 0.2) (layer "F.Cu") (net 19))
 (segment (start 218.52 68.21) (end 216.46 66.15) (width 0.2) (layer "F.Cu") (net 19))
 (segment (start 218.52 91.68) (end 218.52 68.21) (width 0.2) (layer "F.Cu") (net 19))
 (segment (start 214.73887 69.839) (end 214.14113 69.839) (width 0.2) (layer "F.Cu") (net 19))
 (segment (start 191.46 91.675) (end 191.46 95.855) (width 0.2) (layer "F.Cu") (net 19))
 (segment (start 183.25 76.65) (end 181.84 78.06) (width 0.2) (layer "F.Cu") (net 19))
 (segment (start 175.5 78.06) (end 172.939 78.06) (width 0.2) (layer "F.Cu") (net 19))
 (segment (start 172.849 85.969) (end 172.849 80.02) (width 0.2) (layer "F.Cu") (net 19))
 (segment (start 208.29 79.17) (end 210.92 76.54) (width 0.2) (layer "F.Cu") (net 19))
 (segment (start 207.85 88.15) (end 206.73 87.03) (width 0.2) (layer "F.Cu") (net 19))
 (segment (start 198.98 91.1) (end 200.96 89.12) (width 0.2) (layer "F.Cu") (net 19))
 (segment (start 174.15 76.65) (end 183.25 76.65) (width 0.2) (layer "F.Cu") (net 19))
 (segment (start 181.84 78.06) (end 175.5 78.06) (width 0.2) (layer "F.Cu") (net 19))
 (segment (start 206.73 87.03) (end 206.73 80.64) (width 0.2) (layer "F.Cu") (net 19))
 (segment (start 200.96 89.12) (end 203.59 89.12) (width 0.2) (layer "F.Cu") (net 19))
 (segment (start 175.5 78.06) (end 174.809 78.06) (width 0.2) (layer "F.Cu") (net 19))
 (segment (start 213.39487 88.15) (end 207.85 88.15) (width 0.2) (layer "F.Cu") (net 19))
 (segment (start 174.2 87.32) (end 172.849 85.969) (width 0.2) (layer "F.Cu") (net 19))
 (segment (start 172.939 78.06) (end 172.849 78.15) (width 0.2) (layer "F.Cu") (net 19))
 (segment (start 172.849 77.951) (end 174.15 76.65) (width 0.2) (layer "F.Cu") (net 19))
 (segment (start 174.2 90.46) (end 174.41 90.67) (width 0.2) (layer "F.Cu") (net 19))
 (segment (start 193.035 83.378) (end 193.035 83.91) (width 0.2) (layer "F.Cu") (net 19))
 (segment (start 210.92 73.06013) (end 210.92 76.54) (width 0.2) (layer "F.Cu") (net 19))
 (segment (start 192.035 91.1) (end 191.46 91.675) (width 0.2) (layer "F.Cu") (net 19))
 (segment (start 208.02 79.44) (end 208.29 79.17) (width 0.2) (layer "F.Cu") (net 19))
 (segment (start 208.02 87.31) (end 208.02 79.44) (width 0.2) (layer "F.Cu") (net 19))
 (segment (start 213.01 73.76) (end 210.92 75.85) (width 0.2) (layer "F.Cu") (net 19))
 (segment (start 215.08 70.34) (end 215.08 70.18013) (width 0.2) (layer "F.Cu") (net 19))
 (segment (start 187.165 89.23) (end 187.165 89.429999) (width 0.2) (layer "F.Cu") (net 19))
 (segment (start 210.92 75.85) (end 210.92 76.54) (width 0.2) (layer "F.Cu") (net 19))
 (segment (start 215.08 70.18013) (end 214.73887 69.839) (width 0.2) (layer "F.Cu") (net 19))
 (segment (start 183.3 87.32) (end 186.65 90.67) (width 0.2) (layer "F.Cu") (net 19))
 (segment (start 174.41 90.67) (end 186.65 90.67) (width 0.2) (layer "F.Cu") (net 19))
 (segment (start 208.091 87.381) (end 208.02 87.31) (width 0.2) (layer "F.Cu") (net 19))
 (segment (start 192.58 91.1) (end 192.035 91.1) (width 0.2) (layer "F.Cu") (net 19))
 (segment (start 216.46 66.15) (end 204.96 66.15) (width 0.2) (layer "F.Cu") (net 19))
 (segment (start 207.17 92.7) (end 217.5 92.7) (width 0.2) (layer "F.Cu") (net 19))
 (segment (start 174.2 87.32) (end 174.2 90.46) (width 0.2) (layer "F.Cu") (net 19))
 (segment (start 208.2 79.17) (end 208.29 79.17) (width 0.2) (layer "F.Cu") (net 19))
 (segment (start 189.410001 91.675) (end 191.46 91.675) (width 0.2) (layer "F.Cu") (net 19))
 (segment (start 214.475 87.06987) (end 213.39487 88.15) (width 0.2) (layer "F.Cu") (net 19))
 (segment (start 174.809 78.06) (end 172.849 80.02) (width 0.2) (layer "F.Cu") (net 19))
 (segment (start 209.285 87.03987) (end 208.94387 87.381) (width 0.2) (layer "F.Cu") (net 19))
 (segment (start 187.655 91.675) (end 191.46 91.675) (width 0.2) (layer "F.Cu") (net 19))
 (segment (start 203.59 89.12) (end 207.17 92.7) (width 0.2) (layer "F.Cu") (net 19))
 (segment (start 186.65 90.67) (end 187.655 91.675) (width 0.2) (layer "F.Cu") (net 19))
 (segment (start 214.475 86.91) (end 214.475 87.06987) (width 0.2) (layer "F.Cu") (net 19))
 (segment (start 196.403 80.01) (end 193.035 83.378) (width 0.2) (layer "F.Cu") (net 19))
 (segment (start 172.849 80.02) (end 172.849 78.15) (width 0.2) (layer "F.Cu") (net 19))
 (segment (start 174.2 87.32) (end 183.3 87.32) (width 0.2) (layer "F.Cu") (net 19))
 (segment (start 200.1 95.855) (end 191.46 95.855) (width 0.2) (layer "F.Cu") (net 19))
 (segment (start 206.73 80.64) (end 208.2 79.17) (width 0.2) (layer "F.Cu") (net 19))
 (segment (start 208.94387 87.381) (end 208.091 87.381) (width 0.2) (layer "F.Cu") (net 19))
 (segment (start 217.5 92.7) (end 218.52 91.68) (width 0.2) (layer "F.Cu") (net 19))
 (segment (start 172.849 78.15) (end 172.849 77.951) (width 0.2) (layer "F.Cu") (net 19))
 (via (at 197.24 80.01) (size 0.6) (drill 0.3) (layers "F.Cu" "B.Cu") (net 19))
 (segment (start 210.97 93.74) (end 197.24 80.01) (width 0.2) (layer "B.Cu") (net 19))
 (segment (start 210.97 95.37) (end 210.97 93.74) (width 0.2) (layer "B.Cu") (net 19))
 (via (at 187.54 74.97) (size 0.6) (drill 0.3) (layers "F.Cu" "B.Cu") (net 9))
 (segment (start 183.5 77.44) (end 185.97 74.97) (width 0.2) (layer "B.Cu") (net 9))
 (segment (start 185.97 74.97) (end 187.54 74.97) (width 0.2) (layer "B.Cu") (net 9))
 (segment (start 183.5 95.47) (end 183.5 77.44) (width 0.2) (layer "B.Cu") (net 9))
 (via (at 187.59 71.3) (size 0.6) (drill 0.3) (layers "F.Cu" "B.Cu") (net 6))
 (segment (start 187.63 71.34) (end 187.59 71.3) (width 0.2) (layer "B.Cu") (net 6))
 (segment (start 180.5 95.47) (end 180.5 74.24) (width 0.2) (layer "B.Cu") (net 6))
 (segment (start 183.44 71.3) (end 187.59 71.3) (width 0.2) (layer "B.Cu") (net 6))
 (segment (start 180.5 74.24) (end 183.44 71.3) (width 0.2) (layer "B.Cu") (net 6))
 (via (at 187.44 73.87) (size 0.6) (drill 0.3) (layers "F.Cu" "B.Cu") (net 8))
 (segment (start 182.5 95.47) (end 182.5 76.44) (width 0.2) (layer "B.Cu") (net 8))
 (segment (start 185.15 73.87) (end 187.44 73.87) (width 0.2) (layer "B.Cu") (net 8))
 (segment (start 182.5 76.44) (end 185.11 73.83) (width 0.2) (layer "B.Cu") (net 8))
 (segment (start 185.11 73.83) (end 185.15 73.87) (width 0.2) (layer "B.Cu") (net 8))
 (via (at 187.46 69.96) (size 0.6) (drill 0.3) (layers "F.Cu" "B.Cu") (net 5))
 (segment (start 179.5 95.47) (end 179.5 73.32) (width 0.2) (layer "B.Cu") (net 5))
 (segment (start 187.87 69.82) (end 187.6 69.82) (width 0.2) (layer "B.Cu") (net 5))
 (segment (start 187.6 69.82) (end 187.46 69.96) (width 0.2) (layer "B.Cu") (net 5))
 (segment (start 187.73 69.96) (end 187.87 69.82) (width 0.2) (layer "B.Cu") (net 5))
 (segment (start 179.5 73.32) (end 182.86 69.96) (width 0.2) (layer "B.Cu") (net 5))
 (segment (start 182.86 69.96) (end 187.73 69.96) (width 0.2) (layer "B.Cu") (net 5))
 (via (at 187.46 80.12) (size 0.6) (drill 0.3) (layers "F.Cu" "B.Cu") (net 13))
 (segment (start 185.5 81.71) (end 187.27 79.94) (width 0.2) (layer "B.Cu") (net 13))
 (segment (start 185.5 95.47) (end 185.5 81.71) (width 0.2) (layer "B.Cu") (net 13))
 (segment (start 187.45 80.12) (end 187.46 80.12) (width 0.2) (layer "B.Cu") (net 13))
 (segment (start 187.27 79.94) (end 187.45 80.12) (width 0.2) (layer "B.Cu") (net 13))
 (via (at 187.54 72.39) (size 0.6) (drill 0.3) (layers "F.Cu" "B.Cu") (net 7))
 (segment (start 181.5 75.05) (end 184.06 72.49) (width 0.2) (layer "B.Cu") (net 7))
 (segment (start 184.06 72.49) (end 187.44 72.49) (width 0.2) (layer "B.Cu") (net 7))
 (segment (start 181.5 95.47) (end 181.5 75.05) (width 0.2) (layer "B.Cu") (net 7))
 (segment (start 187.44 72.49) (end 187.54 72.39) (width 0.2) (layer "B.Cu") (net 7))
 (via (at 187.46 76.31) (size 0.6) (drill 0.3) (layers "F.Cu" "B.Cu") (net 10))
 (segment (start 186.58 76.21) (end 187.36 76.21) (width 0.2) (layer "B.Cu") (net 10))
 (segment (start 184.5 95.47) (end 184.5 78.29) (width 0.2) (layer "B.Cu") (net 10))
 (segment (start 184.5 78.29) (end 186.58 76.21) (width 0.2) (layer "B.Cu") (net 10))
 (segment (start 187.36 76.21) (end 187.46 76.31) (width 0.2) (layer "B.Cu") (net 10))
 (via (at 189.17 83.85) (size 0.6) (drill 0.3) (layers "F.Cu" "B.Cu") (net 16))
 (segment (start 186.5 95.47) (end 186.5 86.52) (width 0.2) (layer "B.Cu") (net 16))
 (segment (start 186.5 86.52) (end 189.17 83.85) (width 0.2) (layer "B.Cu") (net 16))
 (segment (start 200.433 81.06) (end 198.115 83.378) (width 0.2) (layer "F.Cu") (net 23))
 (segment (start 198.115 83.378) (end 198.115 83.91) (width 0.2) (layer "F.Cu") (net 23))
 (segment (start 201.18 81.06) (end 200.433 81.06) (width 0.2) (layer "F.Cu") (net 23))
 (via (at 201.18 81.06) (size 0.6) (drill 0.3) (layers "F.Cu" "B.Cu") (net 23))
 (segment (start 212.97 95.37) (end 212.97 92.85) (width 0.2) (layer "B.Cu") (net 23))
 (segment (start 212.97 92.85) (end 201.18 81.06) (width 0.2) (layer "B.Cu") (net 23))
 (segment (start 199.413 80.81) (end 196.845 83.378) (width 0.2) (layer "F.Cu") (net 22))
 (segment (start 196.845 83.378) (end 196.845 83.91) (width 0.2) (layer "F.Cu") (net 22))
 (segment (start 199.81 80.81) (end 199.413 80.81) (width 0.2) (layer "F.Cu") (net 22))
 (via (at 199.81 80.81) (size 0.6) (drill 0.3) (layers "F.Cu" "B.Cu") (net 22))
 (segment (start 211.97 92.97) (end 199.81 80.81) (width 0.2) (layer "B.Cu") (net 22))
 (segment (start 211.97 95.37) (end 211.97 92.97) (width 0.2) (layer "B.Cu") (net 22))
 (via (at 187.7 78.83) (size 0.6) (drill 0.3) (layers "F.Cu" "B.Cu") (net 12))
 (segment (start 207.97 95.37) (end 207.97 95.34328) (width 0.2) (layer "B.Cu") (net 12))
 (segment (start 191.45672 78.83) (end 187.7 78.83) (width 0.2) (layer "B.Cu") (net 12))
 (segment (start 207.97 95.34328) (end 191.45672 78.83) (width 0.2) (layer "B.Cu") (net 12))
 (segment (start 187.86 77.58) (end 187.46 77.58) (width 0.2) (layer "F.Cu") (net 11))
 (segment (start 190.22 79.94) (end 187.86 77.58) (width 0.2) (layer "F.Cu") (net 11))
 (via (at 187.46 77.58) (size 0.6) (drill 0.3) (layers "F.Cu" "B.Cu") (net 11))
 (via (at 190.22 79.94) (size 0.6) (drill 0.3) (layers "F.Cu" "B.Cu") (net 11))
 (segment (start 206.97 95.37) (end 205.65 95.37) (width 0.2) (layer "B.Cu") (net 11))
 (segment (start 205.65 95.37) (end 190.22 79.94) (width 0.2) (layer "B.Cu") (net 11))
 (segment (start 202.743 81.29) (end 200.655 83.378) (width 0.2) (layer "F.Cu") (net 25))
 (segment (start 202.99 81.29) (end 202.743 81.29) (width 0.2) (layer "F.Cu") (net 25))
 (segment (start 200.655 83.378) (end 200.655 83.91) (width 0.2) (layer "F.Cu") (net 25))
 (via (at 202.99 81.29) (size 0.6) (drill 0.3) (layers "F.Cu" "B.Cu") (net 25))
 (segment (start 213.97 92.27) (end 202.99 81.29) (width 0.2) (layer "B.Cu") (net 25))
 (segment (start 213.97 95.37) (end 213.97 92.27) (width 0.2) (layer "B.Cu") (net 25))
 (segment (start 195.44 79.78) (end 191.765 83.455) (width 0.2) (layer "F.Cu") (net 18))
 (segment (start 191.765 83.455) (end 191.765 83.91) (width 0.2) (layer "F.Cu") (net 18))
 (via (at 195.44 79.78) (size 0.6) (drill 0.3) (layers "F.Cu" "B.Cu") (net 18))
 (segment (start 209.97 95.37) (end 209.97 94.31) (width 0.2) (layer "B.Cu") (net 18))
 (segment (start 209.97 94.31) (end 195.44 79.78) (width 0.2) (layer "B.Cu") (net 18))
 (segment (start 190.495 82.885) (end 190.495 83.91) (width 0.2) (layer "F.Cu") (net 17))
 (segment (start 193.73 79.65) (end 190.495 82.885) (width 0.2) (layer "F.Cu") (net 17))
 (via (at 193.73 79.65) (size 0.6) (drill 0.3) (layers "F.Cu" "B.Cu") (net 17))
 (segment (start 208.97 94.76896) (end 194.22104 80.02) (width 0.2) (layer "B.Cu") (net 17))
 (segment (start 208.97 95.37) (end 208.97 94.76896) (width 0.2) (layer "B.Cu") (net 17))
 (segment (start 194.22104 80.02) (end 194.21 80.02) (width 0.2) (layer "B.Cu") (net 17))
 (segment (start 194.21 80.02) (end 193.84 79.65) (width 0.2) (layer "B.Cu") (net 17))
 (segment (start 193.84 79.65) (end 193.73 79.65) (width 0.2) (layer "B.Cu") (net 17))
 (segment (start 201.73 66.15) (end 204.559 66.15) (width 0.2) (layer "F.Cu") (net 4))
 (segment (start 188.114264 66.15) (end 187.46 66.15) (width 0.2) (layer "F.Cu") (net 4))
 (segment (start 194.01 72.045736) (end 188.114264 66.15) (width 0.2) (layer "F.Cu") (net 4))
 (segment (start 195.41 72.47) (end 201.73 66.15) (width 0.2) (layer "F.Cu") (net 4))
 (segment (start 194.01 72.47) (end 194.01 72.045736) (width 0.2) (layer "F.Cu") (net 4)))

